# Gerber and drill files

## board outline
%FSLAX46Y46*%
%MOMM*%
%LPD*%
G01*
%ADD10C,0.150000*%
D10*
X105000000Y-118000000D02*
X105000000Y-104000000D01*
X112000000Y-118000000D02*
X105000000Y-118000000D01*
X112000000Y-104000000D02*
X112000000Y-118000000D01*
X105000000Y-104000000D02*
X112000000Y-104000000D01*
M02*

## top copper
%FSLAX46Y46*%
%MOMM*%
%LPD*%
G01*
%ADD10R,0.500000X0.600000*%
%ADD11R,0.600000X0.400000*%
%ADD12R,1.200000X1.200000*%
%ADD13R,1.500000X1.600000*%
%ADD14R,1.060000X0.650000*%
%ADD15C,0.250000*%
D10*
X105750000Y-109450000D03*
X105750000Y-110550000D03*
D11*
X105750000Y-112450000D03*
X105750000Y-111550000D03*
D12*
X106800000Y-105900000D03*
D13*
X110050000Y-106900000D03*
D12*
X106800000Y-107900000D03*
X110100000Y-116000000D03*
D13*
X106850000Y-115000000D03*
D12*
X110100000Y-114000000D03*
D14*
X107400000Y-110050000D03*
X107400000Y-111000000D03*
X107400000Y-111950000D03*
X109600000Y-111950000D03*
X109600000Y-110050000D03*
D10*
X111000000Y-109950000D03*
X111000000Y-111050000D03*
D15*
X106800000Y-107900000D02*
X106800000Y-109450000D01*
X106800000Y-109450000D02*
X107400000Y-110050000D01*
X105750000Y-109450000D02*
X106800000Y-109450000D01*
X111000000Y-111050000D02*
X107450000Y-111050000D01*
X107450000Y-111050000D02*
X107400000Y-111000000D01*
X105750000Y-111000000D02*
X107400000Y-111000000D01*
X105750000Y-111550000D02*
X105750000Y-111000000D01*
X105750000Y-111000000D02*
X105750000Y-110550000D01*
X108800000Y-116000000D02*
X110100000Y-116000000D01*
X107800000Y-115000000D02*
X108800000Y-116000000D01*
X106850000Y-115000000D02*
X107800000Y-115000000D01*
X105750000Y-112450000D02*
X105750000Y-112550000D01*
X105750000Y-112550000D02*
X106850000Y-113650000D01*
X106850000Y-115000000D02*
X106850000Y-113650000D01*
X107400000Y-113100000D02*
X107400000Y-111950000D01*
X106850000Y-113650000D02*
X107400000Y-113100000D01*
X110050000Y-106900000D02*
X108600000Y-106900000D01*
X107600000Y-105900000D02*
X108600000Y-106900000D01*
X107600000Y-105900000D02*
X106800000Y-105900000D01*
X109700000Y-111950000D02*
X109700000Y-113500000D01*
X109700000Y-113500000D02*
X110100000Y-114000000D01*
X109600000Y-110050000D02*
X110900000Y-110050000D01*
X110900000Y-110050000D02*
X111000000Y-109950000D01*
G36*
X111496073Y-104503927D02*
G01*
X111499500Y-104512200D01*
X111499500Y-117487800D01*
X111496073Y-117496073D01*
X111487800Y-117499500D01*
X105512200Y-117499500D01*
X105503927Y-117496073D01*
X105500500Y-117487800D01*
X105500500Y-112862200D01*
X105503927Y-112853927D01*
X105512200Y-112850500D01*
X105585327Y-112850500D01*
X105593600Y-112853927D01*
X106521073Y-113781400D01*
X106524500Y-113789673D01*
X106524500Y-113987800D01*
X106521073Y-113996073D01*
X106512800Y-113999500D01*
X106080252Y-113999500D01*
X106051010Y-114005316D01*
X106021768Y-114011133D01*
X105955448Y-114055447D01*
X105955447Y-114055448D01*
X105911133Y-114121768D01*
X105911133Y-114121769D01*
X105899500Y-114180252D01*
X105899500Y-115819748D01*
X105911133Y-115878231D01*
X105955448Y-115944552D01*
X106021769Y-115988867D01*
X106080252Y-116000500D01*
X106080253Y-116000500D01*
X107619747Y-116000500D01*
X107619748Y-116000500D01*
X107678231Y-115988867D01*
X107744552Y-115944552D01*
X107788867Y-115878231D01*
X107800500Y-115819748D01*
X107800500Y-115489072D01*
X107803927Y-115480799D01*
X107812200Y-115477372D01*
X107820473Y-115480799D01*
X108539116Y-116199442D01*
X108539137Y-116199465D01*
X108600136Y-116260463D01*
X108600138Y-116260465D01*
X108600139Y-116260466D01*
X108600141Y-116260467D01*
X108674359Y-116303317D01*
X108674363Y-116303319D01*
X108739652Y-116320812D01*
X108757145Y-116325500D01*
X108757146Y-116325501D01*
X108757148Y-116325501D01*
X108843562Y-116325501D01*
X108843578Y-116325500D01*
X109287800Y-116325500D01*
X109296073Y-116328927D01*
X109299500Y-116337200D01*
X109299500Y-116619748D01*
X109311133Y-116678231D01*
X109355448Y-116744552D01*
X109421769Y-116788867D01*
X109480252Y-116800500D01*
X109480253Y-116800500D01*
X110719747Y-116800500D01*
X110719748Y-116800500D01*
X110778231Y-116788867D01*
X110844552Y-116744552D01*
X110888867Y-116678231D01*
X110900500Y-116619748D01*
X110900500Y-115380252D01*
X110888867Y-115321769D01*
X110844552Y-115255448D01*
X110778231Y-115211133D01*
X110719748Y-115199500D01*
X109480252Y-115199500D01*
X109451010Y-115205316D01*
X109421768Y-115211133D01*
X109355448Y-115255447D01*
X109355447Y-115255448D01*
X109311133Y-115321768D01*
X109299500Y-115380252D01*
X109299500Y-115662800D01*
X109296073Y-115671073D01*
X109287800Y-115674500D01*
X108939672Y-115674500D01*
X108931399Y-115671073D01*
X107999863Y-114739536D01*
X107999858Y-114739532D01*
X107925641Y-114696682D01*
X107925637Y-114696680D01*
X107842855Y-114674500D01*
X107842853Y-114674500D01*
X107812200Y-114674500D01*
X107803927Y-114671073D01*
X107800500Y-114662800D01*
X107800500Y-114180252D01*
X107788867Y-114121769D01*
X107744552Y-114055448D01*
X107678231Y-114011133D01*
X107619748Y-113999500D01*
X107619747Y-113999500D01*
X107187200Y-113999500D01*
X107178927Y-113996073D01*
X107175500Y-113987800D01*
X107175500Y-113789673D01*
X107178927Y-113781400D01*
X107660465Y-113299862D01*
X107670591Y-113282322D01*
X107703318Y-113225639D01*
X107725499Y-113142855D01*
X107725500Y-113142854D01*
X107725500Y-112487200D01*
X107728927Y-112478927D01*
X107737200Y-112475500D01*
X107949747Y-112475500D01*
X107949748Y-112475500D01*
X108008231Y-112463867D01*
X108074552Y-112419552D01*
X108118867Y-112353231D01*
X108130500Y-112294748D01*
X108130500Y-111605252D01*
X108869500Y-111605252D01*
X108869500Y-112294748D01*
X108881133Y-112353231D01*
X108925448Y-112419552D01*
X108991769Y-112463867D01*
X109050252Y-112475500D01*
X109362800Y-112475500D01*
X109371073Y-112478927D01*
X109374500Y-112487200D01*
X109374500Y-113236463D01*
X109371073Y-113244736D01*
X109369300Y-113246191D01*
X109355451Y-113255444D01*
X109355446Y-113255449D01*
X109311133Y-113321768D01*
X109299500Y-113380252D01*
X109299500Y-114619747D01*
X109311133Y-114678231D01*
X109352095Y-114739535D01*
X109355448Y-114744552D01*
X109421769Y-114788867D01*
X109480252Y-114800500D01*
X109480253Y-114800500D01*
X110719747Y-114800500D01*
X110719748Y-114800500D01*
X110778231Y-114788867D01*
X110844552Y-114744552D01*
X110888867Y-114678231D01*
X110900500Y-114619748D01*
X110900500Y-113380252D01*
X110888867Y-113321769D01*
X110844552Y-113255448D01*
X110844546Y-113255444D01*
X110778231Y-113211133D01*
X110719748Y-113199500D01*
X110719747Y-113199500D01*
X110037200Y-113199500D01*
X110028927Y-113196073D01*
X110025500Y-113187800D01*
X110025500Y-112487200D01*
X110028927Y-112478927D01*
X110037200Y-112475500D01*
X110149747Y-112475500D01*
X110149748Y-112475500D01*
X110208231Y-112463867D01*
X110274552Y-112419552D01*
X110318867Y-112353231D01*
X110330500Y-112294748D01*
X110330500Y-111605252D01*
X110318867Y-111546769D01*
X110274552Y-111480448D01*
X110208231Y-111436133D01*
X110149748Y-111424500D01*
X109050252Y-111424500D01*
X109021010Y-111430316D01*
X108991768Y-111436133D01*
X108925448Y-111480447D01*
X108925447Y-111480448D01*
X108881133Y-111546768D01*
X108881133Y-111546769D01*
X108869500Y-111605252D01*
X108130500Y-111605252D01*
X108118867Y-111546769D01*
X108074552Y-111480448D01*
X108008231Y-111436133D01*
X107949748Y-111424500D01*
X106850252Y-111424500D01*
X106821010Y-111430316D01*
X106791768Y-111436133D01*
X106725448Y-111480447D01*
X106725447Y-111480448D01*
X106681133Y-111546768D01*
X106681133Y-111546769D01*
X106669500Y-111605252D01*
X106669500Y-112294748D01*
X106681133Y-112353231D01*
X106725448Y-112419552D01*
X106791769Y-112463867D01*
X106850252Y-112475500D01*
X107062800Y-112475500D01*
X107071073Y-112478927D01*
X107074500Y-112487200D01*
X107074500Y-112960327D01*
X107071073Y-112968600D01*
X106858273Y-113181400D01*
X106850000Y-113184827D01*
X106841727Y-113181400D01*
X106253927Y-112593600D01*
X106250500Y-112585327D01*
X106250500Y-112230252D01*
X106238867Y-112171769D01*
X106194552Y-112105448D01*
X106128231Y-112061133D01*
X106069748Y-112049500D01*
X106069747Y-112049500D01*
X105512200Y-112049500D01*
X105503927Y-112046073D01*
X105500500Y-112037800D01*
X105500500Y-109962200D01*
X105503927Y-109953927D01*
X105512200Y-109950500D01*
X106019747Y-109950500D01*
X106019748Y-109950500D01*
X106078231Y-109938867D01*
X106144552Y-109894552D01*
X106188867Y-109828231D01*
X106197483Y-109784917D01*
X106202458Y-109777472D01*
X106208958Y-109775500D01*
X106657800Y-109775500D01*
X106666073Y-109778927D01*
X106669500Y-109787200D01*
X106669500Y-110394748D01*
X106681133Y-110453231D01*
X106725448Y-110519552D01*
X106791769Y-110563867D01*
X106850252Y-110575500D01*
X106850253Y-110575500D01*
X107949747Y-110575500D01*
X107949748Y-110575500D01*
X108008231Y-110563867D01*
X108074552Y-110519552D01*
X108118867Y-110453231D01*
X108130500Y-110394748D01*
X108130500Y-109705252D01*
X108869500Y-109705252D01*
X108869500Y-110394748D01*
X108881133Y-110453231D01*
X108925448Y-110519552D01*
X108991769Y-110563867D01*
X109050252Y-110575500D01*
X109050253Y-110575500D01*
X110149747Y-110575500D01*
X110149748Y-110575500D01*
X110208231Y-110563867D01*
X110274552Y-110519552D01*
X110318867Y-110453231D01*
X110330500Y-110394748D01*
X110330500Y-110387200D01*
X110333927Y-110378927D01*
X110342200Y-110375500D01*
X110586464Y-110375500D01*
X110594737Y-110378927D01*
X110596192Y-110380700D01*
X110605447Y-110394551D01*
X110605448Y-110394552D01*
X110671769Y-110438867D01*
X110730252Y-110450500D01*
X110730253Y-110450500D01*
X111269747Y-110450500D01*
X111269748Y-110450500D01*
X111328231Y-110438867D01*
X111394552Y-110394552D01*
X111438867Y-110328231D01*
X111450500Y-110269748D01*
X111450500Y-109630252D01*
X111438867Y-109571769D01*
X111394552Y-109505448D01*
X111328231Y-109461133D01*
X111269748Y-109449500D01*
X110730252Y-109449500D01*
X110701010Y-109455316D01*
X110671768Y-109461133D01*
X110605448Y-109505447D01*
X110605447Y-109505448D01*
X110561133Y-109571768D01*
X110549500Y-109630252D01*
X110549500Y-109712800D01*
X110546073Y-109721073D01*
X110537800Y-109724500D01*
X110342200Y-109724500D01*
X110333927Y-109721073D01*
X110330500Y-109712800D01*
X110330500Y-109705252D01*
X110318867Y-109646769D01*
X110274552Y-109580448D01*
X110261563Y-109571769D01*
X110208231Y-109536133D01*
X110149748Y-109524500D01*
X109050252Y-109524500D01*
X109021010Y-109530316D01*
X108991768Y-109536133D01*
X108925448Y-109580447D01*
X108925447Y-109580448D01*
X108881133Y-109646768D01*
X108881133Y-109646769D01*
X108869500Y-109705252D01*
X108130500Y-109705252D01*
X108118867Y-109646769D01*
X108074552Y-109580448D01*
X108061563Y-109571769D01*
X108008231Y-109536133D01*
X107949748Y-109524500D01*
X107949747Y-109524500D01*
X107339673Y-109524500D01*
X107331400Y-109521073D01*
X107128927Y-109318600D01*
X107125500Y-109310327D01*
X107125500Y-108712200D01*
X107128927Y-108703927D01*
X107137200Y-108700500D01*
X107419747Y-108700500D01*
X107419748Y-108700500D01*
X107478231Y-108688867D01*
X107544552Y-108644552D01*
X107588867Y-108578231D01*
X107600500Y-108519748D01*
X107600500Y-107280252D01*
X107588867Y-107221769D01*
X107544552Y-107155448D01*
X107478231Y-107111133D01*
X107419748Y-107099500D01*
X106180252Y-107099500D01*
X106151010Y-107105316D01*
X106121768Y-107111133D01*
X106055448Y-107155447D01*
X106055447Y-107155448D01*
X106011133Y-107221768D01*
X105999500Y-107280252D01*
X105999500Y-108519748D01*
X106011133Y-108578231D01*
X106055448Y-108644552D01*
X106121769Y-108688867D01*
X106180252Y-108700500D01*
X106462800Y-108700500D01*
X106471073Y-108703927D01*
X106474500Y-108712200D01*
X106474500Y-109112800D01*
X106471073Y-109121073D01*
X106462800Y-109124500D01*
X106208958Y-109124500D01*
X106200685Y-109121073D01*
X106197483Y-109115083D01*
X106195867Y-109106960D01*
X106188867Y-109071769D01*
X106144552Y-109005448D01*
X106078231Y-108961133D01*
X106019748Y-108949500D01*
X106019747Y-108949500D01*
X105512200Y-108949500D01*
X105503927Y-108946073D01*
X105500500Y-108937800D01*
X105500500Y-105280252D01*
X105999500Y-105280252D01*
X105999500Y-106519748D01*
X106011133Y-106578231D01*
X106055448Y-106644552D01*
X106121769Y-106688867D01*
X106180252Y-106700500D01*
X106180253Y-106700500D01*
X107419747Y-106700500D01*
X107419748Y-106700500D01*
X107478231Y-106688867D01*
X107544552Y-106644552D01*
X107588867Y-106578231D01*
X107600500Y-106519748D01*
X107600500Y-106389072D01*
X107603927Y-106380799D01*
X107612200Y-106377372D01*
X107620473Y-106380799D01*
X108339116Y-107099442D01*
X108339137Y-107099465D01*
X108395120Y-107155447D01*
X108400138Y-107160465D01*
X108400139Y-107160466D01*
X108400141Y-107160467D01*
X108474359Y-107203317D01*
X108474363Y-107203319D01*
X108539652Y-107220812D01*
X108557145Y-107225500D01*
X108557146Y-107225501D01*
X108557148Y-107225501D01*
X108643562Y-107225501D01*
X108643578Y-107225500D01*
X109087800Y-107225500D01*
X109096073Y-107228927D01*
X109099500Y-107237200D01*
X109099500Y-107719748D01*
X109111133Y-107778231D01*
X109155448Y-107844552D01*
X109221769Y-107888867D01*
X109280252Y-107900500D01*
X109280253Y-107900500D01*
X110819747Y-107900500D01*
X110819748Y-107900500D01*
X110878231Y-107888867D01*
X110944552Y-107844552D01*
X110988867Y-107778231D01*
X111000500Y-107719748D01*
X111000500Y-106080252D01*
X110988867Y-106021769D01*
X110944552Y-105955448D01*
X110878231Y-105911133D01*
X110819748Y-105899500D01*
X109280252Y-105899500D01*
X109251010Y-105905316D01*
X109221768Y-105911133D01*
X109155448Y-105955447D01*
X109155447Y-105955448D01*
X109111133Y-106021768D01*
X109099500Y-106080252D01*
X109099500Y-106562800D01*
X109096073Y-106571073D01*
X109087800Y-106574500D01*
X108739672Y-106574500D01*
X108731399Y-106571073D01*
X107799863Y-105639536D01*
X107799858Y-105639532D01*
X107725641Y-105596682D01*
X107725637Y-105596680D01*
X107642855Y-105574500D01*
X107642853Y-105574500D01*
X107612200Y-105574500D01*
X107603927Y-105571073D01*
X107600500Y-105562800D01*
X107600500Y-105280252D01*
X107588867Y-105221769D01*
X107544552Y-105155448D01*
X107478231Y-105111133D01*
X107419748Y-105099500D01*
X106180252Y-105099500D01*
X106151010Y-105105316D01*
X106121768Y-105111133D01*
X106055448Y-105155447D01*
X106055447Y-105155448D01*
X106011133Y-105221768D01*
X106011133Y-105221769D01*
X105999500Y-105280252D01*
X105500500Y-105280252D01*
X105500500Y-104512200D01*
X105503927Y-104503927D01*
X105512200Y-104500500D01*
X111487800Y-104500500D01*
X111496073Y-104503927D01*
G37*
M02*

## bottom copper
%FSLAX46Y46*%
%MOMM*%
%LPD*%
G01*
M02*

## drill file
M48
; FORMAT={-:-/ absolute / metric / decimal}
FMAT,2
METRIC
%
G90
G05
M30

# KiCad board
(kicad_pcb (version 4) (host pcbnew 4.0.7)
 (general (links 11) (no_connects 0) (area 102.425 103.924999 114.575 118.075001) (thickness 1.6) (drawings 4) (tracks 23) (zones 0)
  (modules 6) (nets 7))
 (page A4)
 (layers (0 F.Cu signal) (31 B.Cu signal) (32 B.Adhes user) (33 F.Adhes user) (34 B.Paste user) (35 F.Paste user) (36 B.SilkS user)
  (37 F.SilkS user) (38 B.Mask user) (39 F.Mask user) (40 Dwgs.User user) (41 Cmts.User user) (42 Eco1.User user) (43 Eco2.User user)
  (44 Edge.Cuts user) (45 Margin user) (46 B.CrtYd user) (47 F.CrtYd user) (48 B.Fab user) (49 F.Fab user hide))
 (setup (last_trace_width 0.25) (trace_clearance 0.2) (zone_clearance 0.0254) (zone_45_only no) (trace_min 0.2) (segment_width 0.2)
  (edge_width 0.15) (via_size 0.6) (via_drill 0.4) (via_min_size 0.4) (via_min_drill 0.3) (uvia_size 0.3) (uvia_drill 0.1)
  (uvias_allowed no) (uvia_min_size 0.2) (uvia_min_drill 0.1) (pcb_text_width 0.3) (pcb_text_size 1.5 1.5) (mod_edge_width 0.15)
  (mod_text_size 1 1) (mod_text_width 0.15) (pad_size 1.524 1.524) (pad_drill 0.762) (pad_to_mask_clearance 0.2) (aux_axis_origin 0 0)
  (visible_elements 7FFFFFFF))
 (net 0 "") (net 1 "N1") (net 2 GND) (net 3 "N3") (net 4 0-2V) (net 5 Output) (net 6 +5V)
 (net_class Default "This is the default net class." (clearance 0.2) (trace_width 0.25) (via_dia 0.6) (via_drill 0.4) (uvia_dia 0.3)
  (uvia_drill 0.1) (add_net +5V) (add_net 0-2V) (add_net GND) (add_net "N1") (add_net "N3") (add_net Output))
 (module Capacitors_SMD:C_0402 (layer F.Cu) (at 105.75 110 270)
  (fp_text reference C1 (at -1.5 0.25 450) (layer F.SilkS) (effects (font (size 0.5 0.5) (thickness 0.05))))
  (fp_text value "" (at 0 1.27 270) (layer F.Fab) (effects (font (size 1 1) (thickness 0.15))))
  (pad 1 smd rect (at -0.55 0 270) (size 0.6 0.5) (layers F.Cu F.Paste F.Mask) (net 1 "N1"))
  (pad 2 smd rect (at 0.55 0 270) (size 0.6 0.5) (layers F.Cu F.Paste F.Mask) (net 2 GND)))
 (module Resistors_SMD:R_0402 (layer F.Cu) (at 105.75 112 90)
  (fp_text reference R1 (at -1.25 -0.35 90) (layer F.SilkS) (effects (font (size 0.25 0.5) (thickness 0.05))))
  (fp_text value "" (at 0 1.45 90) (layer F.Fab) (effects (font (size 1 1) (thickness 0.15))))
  (pad 1 smd rect (at -0.45 0 90) (size 0.4 0.6) (layers F.Cu F.Paste F.Mask) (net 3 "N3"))
  (pad 2 smd rect (at 0.45 0 90) (size 0.4 0.6) (layers F.Cu F.Paste F.Mask) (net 2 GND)))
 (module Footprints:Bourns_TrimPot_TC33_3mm (layer F.Cu) (at 108.6 106.9 270)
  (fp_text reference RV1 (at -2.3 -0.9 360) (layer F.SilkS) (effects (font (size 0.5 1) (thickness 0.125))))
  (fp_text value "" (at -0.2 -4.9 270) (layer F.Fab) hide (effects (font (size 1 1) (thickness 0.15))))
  (pad 1 smd rect (at -1 1.8 270) (size 1.2 1.2) (layers F.Cu F.Paste F.Mask) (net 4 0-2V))
  (pad 2 smd rect (at 0 -1.45 270) (size 1.6 1.5) (layers F.Cu F.Paste F.Mask) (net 4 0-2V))
  (pad 3 smd rect (at 1 1.8 270) (size 1.2 1.2) (layers F.Cu F.Paste F.Mask) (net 1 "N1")))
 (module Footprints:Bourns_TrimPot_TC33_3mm (layer F.Cu) (at 108.3 115 90)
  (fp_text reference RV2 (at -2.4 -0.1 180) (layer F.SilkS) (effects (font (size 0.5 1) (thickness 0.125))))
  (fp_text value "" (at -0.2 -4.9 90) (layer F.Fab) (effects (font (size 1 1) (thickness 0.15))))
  (pad 1 smd rect (at -1 1.8 90) (size 1.2 1.2) (layers F.Cu F.Paste F.Mask) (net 3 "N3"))
  (pad 2 smd rect (at 0 -1.45 90) (size 1.6 1.5) (layers F.Cu F.Paste F.Mask) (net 3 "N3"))
  (pad 3 smd rect (at 1 1.8 90) (size 1.2 1.2) (layers F.Cu F.Paste F.Mask) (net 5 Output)))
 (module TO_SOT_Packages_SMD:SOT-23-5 (layer F.Cu) (at 108.5 111)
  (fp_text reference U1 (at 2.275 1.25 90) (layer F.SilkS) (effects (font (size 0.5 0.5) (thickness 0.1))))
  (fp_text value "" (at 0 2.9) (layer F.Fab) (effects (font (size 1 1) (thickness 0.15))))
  (pad 1 smd rect (at -1.1 -0.95) (size 1.06 0.65) (layers F.Cu F.Paste F.Mask) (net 1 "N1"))
  (pad 2 smd rect (at -1.1 0) (size 1.06 0.65) (layers F.Cu F.Paste F.Mask) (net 2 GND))
  (pad 3 smd rect (at -1.1 0.95) (size 1.06 0.65) (layers F.Cu F.Paste F.Mask) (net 3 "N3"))
  (pad 4 smd rect (at 1.1 0.95) (size 1.06 0.65) (layers F.Cu F.Paste F.Mask) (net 5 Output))
  (pad 5 smd rect (at 1.1 -0.95) (size 1.06 0.65) (layers F.Cu F.Paste F.Mask) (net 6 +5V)))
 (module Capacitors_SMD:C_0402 (layer F.Cu) (at 111 110.5 270)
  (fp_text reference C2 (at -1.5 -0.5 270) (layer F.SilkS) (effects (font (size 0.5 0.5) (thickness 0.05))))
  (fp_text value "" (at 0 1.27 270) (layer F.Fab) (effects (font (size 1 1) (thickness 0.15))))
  (pad 1 smd rect (at -0.55 0 270) (size 0.6 0.5) (layers F.Cu F.Paste F.Mask) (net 6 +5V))
  (pad 2 smd rect (at 0.55 0 270) (size 0.6 0.5) (layers F.Cu F.Paste F.Mask) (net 2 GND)))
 (gr_line (start 105 118) (end 105 104) (angle 90) (layer Edge.Cuts) (width 0.15))
 (gr_line (start 112 118) (end 105 118) (angle 90) (layer Edge.Cuts) (width 0.15))
 (gr_line (start 112 104) (end 112 118) (angle 90) (layer Edge.Cuts) (width 0.15))
 (gr_line (start 105 104) (end 112 104) (angle 90) (layer Edge.Cuts) (width 0.15))
 (segment (start 106.8 107.9) (end 106.8 109.45) (width 0.25) (layer F.Cu) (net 1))
 (segment (start 106.8 109.45) (end 107.4 110.05) (width 0.25) (layer F.Cu) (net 1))
 (segment (start 105.75 109.45) (end 106.8 109.45) (width 0.25) (layer F.Cu) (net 1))
 (segment (start 111 111.05) (end 107.45 111.05) (width 0.25) (layer F.Cu) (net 2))
 (segment (start 107.45 111.05) (end 107.4 111) (width 0.25) (layer F.Cu) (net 2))
 (segment (start 105.75 111) (end 107.4 111) (width 0.25) (layer F.Cu) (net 2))
 (segment (start 105.75 111.55) (end 105.75 111) (width 0.25) (layer F.Cu) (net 2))
 (segment (start 105.75 111) (end 105.75 110.55) (width 0.25) (layer F.Cu) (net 2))
 (segment (start 108.8 116) (end 110.1 116) (width 0.25) (layer F.Cu) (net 3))
 (segment (start 107.8 115) (end 108.8 116) (width 0.25) (layer F.Cu) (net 3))
 (segment (start 106.85 115) (end 107.8 115) (width 0.25) (layer F.Cu) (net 3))
 (segment (start 105.75 112.45) (end 105.75 112.55) (width 0.25) (layer F.Cu) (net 3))
 (segment (start 105.75 112.55) (end 106.85 113.65) (width 0.25) (layer F.Cu) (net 3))
 (segment (start 106.85 115) (end 106.85 113.65) (width 0.25) (layer F.Cu) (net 3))
 (segment (start 107.4 113.1) (end 107.4 111.95) (width 0.25) (layer F.Cu) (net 3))
 (segment (start 106.85 113.65) (end 107.4 113.1) (width 0.25) (layer F.Cu) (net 3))
 (segment (start 110.05 106.9) (end 108.6 106.9) (width 0.25) (layer F.Cu) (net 4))
 (segment (start 107.6 105.9) (end 108.6 106.9) (width 0.25) (layer F.Cu) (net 4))
 (segment (start 107.6 105.9) (end 106.8 105.9) (width 0.25) (layer F.Cu) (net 4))
 (segment (start 109.7 111.95) (end 109.7 113.5) (width 0.25) (layer F.Cu) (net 5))
 (segment (start 109.7 113.5) (end 110.1 114) (width 0.25) (layer F.Cu) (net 5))
 (segment (start 109.6 110.05) (end 110.9 110.05) (width 0.25) (layer F.Cu) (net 6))
 (segment (start 110.9 110.05) (end 111 109.95) (width 0.25) (layer F.Cu) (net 6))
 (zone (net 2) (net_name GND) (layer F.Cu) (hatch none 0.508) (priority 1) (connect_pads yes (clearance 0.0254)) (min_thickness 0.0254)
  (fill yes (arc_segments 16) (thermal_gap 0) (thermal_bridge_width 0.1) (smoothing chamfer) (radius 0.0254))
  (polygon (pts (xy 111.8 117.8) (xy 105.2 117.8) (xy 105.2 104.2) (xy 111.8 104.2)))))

